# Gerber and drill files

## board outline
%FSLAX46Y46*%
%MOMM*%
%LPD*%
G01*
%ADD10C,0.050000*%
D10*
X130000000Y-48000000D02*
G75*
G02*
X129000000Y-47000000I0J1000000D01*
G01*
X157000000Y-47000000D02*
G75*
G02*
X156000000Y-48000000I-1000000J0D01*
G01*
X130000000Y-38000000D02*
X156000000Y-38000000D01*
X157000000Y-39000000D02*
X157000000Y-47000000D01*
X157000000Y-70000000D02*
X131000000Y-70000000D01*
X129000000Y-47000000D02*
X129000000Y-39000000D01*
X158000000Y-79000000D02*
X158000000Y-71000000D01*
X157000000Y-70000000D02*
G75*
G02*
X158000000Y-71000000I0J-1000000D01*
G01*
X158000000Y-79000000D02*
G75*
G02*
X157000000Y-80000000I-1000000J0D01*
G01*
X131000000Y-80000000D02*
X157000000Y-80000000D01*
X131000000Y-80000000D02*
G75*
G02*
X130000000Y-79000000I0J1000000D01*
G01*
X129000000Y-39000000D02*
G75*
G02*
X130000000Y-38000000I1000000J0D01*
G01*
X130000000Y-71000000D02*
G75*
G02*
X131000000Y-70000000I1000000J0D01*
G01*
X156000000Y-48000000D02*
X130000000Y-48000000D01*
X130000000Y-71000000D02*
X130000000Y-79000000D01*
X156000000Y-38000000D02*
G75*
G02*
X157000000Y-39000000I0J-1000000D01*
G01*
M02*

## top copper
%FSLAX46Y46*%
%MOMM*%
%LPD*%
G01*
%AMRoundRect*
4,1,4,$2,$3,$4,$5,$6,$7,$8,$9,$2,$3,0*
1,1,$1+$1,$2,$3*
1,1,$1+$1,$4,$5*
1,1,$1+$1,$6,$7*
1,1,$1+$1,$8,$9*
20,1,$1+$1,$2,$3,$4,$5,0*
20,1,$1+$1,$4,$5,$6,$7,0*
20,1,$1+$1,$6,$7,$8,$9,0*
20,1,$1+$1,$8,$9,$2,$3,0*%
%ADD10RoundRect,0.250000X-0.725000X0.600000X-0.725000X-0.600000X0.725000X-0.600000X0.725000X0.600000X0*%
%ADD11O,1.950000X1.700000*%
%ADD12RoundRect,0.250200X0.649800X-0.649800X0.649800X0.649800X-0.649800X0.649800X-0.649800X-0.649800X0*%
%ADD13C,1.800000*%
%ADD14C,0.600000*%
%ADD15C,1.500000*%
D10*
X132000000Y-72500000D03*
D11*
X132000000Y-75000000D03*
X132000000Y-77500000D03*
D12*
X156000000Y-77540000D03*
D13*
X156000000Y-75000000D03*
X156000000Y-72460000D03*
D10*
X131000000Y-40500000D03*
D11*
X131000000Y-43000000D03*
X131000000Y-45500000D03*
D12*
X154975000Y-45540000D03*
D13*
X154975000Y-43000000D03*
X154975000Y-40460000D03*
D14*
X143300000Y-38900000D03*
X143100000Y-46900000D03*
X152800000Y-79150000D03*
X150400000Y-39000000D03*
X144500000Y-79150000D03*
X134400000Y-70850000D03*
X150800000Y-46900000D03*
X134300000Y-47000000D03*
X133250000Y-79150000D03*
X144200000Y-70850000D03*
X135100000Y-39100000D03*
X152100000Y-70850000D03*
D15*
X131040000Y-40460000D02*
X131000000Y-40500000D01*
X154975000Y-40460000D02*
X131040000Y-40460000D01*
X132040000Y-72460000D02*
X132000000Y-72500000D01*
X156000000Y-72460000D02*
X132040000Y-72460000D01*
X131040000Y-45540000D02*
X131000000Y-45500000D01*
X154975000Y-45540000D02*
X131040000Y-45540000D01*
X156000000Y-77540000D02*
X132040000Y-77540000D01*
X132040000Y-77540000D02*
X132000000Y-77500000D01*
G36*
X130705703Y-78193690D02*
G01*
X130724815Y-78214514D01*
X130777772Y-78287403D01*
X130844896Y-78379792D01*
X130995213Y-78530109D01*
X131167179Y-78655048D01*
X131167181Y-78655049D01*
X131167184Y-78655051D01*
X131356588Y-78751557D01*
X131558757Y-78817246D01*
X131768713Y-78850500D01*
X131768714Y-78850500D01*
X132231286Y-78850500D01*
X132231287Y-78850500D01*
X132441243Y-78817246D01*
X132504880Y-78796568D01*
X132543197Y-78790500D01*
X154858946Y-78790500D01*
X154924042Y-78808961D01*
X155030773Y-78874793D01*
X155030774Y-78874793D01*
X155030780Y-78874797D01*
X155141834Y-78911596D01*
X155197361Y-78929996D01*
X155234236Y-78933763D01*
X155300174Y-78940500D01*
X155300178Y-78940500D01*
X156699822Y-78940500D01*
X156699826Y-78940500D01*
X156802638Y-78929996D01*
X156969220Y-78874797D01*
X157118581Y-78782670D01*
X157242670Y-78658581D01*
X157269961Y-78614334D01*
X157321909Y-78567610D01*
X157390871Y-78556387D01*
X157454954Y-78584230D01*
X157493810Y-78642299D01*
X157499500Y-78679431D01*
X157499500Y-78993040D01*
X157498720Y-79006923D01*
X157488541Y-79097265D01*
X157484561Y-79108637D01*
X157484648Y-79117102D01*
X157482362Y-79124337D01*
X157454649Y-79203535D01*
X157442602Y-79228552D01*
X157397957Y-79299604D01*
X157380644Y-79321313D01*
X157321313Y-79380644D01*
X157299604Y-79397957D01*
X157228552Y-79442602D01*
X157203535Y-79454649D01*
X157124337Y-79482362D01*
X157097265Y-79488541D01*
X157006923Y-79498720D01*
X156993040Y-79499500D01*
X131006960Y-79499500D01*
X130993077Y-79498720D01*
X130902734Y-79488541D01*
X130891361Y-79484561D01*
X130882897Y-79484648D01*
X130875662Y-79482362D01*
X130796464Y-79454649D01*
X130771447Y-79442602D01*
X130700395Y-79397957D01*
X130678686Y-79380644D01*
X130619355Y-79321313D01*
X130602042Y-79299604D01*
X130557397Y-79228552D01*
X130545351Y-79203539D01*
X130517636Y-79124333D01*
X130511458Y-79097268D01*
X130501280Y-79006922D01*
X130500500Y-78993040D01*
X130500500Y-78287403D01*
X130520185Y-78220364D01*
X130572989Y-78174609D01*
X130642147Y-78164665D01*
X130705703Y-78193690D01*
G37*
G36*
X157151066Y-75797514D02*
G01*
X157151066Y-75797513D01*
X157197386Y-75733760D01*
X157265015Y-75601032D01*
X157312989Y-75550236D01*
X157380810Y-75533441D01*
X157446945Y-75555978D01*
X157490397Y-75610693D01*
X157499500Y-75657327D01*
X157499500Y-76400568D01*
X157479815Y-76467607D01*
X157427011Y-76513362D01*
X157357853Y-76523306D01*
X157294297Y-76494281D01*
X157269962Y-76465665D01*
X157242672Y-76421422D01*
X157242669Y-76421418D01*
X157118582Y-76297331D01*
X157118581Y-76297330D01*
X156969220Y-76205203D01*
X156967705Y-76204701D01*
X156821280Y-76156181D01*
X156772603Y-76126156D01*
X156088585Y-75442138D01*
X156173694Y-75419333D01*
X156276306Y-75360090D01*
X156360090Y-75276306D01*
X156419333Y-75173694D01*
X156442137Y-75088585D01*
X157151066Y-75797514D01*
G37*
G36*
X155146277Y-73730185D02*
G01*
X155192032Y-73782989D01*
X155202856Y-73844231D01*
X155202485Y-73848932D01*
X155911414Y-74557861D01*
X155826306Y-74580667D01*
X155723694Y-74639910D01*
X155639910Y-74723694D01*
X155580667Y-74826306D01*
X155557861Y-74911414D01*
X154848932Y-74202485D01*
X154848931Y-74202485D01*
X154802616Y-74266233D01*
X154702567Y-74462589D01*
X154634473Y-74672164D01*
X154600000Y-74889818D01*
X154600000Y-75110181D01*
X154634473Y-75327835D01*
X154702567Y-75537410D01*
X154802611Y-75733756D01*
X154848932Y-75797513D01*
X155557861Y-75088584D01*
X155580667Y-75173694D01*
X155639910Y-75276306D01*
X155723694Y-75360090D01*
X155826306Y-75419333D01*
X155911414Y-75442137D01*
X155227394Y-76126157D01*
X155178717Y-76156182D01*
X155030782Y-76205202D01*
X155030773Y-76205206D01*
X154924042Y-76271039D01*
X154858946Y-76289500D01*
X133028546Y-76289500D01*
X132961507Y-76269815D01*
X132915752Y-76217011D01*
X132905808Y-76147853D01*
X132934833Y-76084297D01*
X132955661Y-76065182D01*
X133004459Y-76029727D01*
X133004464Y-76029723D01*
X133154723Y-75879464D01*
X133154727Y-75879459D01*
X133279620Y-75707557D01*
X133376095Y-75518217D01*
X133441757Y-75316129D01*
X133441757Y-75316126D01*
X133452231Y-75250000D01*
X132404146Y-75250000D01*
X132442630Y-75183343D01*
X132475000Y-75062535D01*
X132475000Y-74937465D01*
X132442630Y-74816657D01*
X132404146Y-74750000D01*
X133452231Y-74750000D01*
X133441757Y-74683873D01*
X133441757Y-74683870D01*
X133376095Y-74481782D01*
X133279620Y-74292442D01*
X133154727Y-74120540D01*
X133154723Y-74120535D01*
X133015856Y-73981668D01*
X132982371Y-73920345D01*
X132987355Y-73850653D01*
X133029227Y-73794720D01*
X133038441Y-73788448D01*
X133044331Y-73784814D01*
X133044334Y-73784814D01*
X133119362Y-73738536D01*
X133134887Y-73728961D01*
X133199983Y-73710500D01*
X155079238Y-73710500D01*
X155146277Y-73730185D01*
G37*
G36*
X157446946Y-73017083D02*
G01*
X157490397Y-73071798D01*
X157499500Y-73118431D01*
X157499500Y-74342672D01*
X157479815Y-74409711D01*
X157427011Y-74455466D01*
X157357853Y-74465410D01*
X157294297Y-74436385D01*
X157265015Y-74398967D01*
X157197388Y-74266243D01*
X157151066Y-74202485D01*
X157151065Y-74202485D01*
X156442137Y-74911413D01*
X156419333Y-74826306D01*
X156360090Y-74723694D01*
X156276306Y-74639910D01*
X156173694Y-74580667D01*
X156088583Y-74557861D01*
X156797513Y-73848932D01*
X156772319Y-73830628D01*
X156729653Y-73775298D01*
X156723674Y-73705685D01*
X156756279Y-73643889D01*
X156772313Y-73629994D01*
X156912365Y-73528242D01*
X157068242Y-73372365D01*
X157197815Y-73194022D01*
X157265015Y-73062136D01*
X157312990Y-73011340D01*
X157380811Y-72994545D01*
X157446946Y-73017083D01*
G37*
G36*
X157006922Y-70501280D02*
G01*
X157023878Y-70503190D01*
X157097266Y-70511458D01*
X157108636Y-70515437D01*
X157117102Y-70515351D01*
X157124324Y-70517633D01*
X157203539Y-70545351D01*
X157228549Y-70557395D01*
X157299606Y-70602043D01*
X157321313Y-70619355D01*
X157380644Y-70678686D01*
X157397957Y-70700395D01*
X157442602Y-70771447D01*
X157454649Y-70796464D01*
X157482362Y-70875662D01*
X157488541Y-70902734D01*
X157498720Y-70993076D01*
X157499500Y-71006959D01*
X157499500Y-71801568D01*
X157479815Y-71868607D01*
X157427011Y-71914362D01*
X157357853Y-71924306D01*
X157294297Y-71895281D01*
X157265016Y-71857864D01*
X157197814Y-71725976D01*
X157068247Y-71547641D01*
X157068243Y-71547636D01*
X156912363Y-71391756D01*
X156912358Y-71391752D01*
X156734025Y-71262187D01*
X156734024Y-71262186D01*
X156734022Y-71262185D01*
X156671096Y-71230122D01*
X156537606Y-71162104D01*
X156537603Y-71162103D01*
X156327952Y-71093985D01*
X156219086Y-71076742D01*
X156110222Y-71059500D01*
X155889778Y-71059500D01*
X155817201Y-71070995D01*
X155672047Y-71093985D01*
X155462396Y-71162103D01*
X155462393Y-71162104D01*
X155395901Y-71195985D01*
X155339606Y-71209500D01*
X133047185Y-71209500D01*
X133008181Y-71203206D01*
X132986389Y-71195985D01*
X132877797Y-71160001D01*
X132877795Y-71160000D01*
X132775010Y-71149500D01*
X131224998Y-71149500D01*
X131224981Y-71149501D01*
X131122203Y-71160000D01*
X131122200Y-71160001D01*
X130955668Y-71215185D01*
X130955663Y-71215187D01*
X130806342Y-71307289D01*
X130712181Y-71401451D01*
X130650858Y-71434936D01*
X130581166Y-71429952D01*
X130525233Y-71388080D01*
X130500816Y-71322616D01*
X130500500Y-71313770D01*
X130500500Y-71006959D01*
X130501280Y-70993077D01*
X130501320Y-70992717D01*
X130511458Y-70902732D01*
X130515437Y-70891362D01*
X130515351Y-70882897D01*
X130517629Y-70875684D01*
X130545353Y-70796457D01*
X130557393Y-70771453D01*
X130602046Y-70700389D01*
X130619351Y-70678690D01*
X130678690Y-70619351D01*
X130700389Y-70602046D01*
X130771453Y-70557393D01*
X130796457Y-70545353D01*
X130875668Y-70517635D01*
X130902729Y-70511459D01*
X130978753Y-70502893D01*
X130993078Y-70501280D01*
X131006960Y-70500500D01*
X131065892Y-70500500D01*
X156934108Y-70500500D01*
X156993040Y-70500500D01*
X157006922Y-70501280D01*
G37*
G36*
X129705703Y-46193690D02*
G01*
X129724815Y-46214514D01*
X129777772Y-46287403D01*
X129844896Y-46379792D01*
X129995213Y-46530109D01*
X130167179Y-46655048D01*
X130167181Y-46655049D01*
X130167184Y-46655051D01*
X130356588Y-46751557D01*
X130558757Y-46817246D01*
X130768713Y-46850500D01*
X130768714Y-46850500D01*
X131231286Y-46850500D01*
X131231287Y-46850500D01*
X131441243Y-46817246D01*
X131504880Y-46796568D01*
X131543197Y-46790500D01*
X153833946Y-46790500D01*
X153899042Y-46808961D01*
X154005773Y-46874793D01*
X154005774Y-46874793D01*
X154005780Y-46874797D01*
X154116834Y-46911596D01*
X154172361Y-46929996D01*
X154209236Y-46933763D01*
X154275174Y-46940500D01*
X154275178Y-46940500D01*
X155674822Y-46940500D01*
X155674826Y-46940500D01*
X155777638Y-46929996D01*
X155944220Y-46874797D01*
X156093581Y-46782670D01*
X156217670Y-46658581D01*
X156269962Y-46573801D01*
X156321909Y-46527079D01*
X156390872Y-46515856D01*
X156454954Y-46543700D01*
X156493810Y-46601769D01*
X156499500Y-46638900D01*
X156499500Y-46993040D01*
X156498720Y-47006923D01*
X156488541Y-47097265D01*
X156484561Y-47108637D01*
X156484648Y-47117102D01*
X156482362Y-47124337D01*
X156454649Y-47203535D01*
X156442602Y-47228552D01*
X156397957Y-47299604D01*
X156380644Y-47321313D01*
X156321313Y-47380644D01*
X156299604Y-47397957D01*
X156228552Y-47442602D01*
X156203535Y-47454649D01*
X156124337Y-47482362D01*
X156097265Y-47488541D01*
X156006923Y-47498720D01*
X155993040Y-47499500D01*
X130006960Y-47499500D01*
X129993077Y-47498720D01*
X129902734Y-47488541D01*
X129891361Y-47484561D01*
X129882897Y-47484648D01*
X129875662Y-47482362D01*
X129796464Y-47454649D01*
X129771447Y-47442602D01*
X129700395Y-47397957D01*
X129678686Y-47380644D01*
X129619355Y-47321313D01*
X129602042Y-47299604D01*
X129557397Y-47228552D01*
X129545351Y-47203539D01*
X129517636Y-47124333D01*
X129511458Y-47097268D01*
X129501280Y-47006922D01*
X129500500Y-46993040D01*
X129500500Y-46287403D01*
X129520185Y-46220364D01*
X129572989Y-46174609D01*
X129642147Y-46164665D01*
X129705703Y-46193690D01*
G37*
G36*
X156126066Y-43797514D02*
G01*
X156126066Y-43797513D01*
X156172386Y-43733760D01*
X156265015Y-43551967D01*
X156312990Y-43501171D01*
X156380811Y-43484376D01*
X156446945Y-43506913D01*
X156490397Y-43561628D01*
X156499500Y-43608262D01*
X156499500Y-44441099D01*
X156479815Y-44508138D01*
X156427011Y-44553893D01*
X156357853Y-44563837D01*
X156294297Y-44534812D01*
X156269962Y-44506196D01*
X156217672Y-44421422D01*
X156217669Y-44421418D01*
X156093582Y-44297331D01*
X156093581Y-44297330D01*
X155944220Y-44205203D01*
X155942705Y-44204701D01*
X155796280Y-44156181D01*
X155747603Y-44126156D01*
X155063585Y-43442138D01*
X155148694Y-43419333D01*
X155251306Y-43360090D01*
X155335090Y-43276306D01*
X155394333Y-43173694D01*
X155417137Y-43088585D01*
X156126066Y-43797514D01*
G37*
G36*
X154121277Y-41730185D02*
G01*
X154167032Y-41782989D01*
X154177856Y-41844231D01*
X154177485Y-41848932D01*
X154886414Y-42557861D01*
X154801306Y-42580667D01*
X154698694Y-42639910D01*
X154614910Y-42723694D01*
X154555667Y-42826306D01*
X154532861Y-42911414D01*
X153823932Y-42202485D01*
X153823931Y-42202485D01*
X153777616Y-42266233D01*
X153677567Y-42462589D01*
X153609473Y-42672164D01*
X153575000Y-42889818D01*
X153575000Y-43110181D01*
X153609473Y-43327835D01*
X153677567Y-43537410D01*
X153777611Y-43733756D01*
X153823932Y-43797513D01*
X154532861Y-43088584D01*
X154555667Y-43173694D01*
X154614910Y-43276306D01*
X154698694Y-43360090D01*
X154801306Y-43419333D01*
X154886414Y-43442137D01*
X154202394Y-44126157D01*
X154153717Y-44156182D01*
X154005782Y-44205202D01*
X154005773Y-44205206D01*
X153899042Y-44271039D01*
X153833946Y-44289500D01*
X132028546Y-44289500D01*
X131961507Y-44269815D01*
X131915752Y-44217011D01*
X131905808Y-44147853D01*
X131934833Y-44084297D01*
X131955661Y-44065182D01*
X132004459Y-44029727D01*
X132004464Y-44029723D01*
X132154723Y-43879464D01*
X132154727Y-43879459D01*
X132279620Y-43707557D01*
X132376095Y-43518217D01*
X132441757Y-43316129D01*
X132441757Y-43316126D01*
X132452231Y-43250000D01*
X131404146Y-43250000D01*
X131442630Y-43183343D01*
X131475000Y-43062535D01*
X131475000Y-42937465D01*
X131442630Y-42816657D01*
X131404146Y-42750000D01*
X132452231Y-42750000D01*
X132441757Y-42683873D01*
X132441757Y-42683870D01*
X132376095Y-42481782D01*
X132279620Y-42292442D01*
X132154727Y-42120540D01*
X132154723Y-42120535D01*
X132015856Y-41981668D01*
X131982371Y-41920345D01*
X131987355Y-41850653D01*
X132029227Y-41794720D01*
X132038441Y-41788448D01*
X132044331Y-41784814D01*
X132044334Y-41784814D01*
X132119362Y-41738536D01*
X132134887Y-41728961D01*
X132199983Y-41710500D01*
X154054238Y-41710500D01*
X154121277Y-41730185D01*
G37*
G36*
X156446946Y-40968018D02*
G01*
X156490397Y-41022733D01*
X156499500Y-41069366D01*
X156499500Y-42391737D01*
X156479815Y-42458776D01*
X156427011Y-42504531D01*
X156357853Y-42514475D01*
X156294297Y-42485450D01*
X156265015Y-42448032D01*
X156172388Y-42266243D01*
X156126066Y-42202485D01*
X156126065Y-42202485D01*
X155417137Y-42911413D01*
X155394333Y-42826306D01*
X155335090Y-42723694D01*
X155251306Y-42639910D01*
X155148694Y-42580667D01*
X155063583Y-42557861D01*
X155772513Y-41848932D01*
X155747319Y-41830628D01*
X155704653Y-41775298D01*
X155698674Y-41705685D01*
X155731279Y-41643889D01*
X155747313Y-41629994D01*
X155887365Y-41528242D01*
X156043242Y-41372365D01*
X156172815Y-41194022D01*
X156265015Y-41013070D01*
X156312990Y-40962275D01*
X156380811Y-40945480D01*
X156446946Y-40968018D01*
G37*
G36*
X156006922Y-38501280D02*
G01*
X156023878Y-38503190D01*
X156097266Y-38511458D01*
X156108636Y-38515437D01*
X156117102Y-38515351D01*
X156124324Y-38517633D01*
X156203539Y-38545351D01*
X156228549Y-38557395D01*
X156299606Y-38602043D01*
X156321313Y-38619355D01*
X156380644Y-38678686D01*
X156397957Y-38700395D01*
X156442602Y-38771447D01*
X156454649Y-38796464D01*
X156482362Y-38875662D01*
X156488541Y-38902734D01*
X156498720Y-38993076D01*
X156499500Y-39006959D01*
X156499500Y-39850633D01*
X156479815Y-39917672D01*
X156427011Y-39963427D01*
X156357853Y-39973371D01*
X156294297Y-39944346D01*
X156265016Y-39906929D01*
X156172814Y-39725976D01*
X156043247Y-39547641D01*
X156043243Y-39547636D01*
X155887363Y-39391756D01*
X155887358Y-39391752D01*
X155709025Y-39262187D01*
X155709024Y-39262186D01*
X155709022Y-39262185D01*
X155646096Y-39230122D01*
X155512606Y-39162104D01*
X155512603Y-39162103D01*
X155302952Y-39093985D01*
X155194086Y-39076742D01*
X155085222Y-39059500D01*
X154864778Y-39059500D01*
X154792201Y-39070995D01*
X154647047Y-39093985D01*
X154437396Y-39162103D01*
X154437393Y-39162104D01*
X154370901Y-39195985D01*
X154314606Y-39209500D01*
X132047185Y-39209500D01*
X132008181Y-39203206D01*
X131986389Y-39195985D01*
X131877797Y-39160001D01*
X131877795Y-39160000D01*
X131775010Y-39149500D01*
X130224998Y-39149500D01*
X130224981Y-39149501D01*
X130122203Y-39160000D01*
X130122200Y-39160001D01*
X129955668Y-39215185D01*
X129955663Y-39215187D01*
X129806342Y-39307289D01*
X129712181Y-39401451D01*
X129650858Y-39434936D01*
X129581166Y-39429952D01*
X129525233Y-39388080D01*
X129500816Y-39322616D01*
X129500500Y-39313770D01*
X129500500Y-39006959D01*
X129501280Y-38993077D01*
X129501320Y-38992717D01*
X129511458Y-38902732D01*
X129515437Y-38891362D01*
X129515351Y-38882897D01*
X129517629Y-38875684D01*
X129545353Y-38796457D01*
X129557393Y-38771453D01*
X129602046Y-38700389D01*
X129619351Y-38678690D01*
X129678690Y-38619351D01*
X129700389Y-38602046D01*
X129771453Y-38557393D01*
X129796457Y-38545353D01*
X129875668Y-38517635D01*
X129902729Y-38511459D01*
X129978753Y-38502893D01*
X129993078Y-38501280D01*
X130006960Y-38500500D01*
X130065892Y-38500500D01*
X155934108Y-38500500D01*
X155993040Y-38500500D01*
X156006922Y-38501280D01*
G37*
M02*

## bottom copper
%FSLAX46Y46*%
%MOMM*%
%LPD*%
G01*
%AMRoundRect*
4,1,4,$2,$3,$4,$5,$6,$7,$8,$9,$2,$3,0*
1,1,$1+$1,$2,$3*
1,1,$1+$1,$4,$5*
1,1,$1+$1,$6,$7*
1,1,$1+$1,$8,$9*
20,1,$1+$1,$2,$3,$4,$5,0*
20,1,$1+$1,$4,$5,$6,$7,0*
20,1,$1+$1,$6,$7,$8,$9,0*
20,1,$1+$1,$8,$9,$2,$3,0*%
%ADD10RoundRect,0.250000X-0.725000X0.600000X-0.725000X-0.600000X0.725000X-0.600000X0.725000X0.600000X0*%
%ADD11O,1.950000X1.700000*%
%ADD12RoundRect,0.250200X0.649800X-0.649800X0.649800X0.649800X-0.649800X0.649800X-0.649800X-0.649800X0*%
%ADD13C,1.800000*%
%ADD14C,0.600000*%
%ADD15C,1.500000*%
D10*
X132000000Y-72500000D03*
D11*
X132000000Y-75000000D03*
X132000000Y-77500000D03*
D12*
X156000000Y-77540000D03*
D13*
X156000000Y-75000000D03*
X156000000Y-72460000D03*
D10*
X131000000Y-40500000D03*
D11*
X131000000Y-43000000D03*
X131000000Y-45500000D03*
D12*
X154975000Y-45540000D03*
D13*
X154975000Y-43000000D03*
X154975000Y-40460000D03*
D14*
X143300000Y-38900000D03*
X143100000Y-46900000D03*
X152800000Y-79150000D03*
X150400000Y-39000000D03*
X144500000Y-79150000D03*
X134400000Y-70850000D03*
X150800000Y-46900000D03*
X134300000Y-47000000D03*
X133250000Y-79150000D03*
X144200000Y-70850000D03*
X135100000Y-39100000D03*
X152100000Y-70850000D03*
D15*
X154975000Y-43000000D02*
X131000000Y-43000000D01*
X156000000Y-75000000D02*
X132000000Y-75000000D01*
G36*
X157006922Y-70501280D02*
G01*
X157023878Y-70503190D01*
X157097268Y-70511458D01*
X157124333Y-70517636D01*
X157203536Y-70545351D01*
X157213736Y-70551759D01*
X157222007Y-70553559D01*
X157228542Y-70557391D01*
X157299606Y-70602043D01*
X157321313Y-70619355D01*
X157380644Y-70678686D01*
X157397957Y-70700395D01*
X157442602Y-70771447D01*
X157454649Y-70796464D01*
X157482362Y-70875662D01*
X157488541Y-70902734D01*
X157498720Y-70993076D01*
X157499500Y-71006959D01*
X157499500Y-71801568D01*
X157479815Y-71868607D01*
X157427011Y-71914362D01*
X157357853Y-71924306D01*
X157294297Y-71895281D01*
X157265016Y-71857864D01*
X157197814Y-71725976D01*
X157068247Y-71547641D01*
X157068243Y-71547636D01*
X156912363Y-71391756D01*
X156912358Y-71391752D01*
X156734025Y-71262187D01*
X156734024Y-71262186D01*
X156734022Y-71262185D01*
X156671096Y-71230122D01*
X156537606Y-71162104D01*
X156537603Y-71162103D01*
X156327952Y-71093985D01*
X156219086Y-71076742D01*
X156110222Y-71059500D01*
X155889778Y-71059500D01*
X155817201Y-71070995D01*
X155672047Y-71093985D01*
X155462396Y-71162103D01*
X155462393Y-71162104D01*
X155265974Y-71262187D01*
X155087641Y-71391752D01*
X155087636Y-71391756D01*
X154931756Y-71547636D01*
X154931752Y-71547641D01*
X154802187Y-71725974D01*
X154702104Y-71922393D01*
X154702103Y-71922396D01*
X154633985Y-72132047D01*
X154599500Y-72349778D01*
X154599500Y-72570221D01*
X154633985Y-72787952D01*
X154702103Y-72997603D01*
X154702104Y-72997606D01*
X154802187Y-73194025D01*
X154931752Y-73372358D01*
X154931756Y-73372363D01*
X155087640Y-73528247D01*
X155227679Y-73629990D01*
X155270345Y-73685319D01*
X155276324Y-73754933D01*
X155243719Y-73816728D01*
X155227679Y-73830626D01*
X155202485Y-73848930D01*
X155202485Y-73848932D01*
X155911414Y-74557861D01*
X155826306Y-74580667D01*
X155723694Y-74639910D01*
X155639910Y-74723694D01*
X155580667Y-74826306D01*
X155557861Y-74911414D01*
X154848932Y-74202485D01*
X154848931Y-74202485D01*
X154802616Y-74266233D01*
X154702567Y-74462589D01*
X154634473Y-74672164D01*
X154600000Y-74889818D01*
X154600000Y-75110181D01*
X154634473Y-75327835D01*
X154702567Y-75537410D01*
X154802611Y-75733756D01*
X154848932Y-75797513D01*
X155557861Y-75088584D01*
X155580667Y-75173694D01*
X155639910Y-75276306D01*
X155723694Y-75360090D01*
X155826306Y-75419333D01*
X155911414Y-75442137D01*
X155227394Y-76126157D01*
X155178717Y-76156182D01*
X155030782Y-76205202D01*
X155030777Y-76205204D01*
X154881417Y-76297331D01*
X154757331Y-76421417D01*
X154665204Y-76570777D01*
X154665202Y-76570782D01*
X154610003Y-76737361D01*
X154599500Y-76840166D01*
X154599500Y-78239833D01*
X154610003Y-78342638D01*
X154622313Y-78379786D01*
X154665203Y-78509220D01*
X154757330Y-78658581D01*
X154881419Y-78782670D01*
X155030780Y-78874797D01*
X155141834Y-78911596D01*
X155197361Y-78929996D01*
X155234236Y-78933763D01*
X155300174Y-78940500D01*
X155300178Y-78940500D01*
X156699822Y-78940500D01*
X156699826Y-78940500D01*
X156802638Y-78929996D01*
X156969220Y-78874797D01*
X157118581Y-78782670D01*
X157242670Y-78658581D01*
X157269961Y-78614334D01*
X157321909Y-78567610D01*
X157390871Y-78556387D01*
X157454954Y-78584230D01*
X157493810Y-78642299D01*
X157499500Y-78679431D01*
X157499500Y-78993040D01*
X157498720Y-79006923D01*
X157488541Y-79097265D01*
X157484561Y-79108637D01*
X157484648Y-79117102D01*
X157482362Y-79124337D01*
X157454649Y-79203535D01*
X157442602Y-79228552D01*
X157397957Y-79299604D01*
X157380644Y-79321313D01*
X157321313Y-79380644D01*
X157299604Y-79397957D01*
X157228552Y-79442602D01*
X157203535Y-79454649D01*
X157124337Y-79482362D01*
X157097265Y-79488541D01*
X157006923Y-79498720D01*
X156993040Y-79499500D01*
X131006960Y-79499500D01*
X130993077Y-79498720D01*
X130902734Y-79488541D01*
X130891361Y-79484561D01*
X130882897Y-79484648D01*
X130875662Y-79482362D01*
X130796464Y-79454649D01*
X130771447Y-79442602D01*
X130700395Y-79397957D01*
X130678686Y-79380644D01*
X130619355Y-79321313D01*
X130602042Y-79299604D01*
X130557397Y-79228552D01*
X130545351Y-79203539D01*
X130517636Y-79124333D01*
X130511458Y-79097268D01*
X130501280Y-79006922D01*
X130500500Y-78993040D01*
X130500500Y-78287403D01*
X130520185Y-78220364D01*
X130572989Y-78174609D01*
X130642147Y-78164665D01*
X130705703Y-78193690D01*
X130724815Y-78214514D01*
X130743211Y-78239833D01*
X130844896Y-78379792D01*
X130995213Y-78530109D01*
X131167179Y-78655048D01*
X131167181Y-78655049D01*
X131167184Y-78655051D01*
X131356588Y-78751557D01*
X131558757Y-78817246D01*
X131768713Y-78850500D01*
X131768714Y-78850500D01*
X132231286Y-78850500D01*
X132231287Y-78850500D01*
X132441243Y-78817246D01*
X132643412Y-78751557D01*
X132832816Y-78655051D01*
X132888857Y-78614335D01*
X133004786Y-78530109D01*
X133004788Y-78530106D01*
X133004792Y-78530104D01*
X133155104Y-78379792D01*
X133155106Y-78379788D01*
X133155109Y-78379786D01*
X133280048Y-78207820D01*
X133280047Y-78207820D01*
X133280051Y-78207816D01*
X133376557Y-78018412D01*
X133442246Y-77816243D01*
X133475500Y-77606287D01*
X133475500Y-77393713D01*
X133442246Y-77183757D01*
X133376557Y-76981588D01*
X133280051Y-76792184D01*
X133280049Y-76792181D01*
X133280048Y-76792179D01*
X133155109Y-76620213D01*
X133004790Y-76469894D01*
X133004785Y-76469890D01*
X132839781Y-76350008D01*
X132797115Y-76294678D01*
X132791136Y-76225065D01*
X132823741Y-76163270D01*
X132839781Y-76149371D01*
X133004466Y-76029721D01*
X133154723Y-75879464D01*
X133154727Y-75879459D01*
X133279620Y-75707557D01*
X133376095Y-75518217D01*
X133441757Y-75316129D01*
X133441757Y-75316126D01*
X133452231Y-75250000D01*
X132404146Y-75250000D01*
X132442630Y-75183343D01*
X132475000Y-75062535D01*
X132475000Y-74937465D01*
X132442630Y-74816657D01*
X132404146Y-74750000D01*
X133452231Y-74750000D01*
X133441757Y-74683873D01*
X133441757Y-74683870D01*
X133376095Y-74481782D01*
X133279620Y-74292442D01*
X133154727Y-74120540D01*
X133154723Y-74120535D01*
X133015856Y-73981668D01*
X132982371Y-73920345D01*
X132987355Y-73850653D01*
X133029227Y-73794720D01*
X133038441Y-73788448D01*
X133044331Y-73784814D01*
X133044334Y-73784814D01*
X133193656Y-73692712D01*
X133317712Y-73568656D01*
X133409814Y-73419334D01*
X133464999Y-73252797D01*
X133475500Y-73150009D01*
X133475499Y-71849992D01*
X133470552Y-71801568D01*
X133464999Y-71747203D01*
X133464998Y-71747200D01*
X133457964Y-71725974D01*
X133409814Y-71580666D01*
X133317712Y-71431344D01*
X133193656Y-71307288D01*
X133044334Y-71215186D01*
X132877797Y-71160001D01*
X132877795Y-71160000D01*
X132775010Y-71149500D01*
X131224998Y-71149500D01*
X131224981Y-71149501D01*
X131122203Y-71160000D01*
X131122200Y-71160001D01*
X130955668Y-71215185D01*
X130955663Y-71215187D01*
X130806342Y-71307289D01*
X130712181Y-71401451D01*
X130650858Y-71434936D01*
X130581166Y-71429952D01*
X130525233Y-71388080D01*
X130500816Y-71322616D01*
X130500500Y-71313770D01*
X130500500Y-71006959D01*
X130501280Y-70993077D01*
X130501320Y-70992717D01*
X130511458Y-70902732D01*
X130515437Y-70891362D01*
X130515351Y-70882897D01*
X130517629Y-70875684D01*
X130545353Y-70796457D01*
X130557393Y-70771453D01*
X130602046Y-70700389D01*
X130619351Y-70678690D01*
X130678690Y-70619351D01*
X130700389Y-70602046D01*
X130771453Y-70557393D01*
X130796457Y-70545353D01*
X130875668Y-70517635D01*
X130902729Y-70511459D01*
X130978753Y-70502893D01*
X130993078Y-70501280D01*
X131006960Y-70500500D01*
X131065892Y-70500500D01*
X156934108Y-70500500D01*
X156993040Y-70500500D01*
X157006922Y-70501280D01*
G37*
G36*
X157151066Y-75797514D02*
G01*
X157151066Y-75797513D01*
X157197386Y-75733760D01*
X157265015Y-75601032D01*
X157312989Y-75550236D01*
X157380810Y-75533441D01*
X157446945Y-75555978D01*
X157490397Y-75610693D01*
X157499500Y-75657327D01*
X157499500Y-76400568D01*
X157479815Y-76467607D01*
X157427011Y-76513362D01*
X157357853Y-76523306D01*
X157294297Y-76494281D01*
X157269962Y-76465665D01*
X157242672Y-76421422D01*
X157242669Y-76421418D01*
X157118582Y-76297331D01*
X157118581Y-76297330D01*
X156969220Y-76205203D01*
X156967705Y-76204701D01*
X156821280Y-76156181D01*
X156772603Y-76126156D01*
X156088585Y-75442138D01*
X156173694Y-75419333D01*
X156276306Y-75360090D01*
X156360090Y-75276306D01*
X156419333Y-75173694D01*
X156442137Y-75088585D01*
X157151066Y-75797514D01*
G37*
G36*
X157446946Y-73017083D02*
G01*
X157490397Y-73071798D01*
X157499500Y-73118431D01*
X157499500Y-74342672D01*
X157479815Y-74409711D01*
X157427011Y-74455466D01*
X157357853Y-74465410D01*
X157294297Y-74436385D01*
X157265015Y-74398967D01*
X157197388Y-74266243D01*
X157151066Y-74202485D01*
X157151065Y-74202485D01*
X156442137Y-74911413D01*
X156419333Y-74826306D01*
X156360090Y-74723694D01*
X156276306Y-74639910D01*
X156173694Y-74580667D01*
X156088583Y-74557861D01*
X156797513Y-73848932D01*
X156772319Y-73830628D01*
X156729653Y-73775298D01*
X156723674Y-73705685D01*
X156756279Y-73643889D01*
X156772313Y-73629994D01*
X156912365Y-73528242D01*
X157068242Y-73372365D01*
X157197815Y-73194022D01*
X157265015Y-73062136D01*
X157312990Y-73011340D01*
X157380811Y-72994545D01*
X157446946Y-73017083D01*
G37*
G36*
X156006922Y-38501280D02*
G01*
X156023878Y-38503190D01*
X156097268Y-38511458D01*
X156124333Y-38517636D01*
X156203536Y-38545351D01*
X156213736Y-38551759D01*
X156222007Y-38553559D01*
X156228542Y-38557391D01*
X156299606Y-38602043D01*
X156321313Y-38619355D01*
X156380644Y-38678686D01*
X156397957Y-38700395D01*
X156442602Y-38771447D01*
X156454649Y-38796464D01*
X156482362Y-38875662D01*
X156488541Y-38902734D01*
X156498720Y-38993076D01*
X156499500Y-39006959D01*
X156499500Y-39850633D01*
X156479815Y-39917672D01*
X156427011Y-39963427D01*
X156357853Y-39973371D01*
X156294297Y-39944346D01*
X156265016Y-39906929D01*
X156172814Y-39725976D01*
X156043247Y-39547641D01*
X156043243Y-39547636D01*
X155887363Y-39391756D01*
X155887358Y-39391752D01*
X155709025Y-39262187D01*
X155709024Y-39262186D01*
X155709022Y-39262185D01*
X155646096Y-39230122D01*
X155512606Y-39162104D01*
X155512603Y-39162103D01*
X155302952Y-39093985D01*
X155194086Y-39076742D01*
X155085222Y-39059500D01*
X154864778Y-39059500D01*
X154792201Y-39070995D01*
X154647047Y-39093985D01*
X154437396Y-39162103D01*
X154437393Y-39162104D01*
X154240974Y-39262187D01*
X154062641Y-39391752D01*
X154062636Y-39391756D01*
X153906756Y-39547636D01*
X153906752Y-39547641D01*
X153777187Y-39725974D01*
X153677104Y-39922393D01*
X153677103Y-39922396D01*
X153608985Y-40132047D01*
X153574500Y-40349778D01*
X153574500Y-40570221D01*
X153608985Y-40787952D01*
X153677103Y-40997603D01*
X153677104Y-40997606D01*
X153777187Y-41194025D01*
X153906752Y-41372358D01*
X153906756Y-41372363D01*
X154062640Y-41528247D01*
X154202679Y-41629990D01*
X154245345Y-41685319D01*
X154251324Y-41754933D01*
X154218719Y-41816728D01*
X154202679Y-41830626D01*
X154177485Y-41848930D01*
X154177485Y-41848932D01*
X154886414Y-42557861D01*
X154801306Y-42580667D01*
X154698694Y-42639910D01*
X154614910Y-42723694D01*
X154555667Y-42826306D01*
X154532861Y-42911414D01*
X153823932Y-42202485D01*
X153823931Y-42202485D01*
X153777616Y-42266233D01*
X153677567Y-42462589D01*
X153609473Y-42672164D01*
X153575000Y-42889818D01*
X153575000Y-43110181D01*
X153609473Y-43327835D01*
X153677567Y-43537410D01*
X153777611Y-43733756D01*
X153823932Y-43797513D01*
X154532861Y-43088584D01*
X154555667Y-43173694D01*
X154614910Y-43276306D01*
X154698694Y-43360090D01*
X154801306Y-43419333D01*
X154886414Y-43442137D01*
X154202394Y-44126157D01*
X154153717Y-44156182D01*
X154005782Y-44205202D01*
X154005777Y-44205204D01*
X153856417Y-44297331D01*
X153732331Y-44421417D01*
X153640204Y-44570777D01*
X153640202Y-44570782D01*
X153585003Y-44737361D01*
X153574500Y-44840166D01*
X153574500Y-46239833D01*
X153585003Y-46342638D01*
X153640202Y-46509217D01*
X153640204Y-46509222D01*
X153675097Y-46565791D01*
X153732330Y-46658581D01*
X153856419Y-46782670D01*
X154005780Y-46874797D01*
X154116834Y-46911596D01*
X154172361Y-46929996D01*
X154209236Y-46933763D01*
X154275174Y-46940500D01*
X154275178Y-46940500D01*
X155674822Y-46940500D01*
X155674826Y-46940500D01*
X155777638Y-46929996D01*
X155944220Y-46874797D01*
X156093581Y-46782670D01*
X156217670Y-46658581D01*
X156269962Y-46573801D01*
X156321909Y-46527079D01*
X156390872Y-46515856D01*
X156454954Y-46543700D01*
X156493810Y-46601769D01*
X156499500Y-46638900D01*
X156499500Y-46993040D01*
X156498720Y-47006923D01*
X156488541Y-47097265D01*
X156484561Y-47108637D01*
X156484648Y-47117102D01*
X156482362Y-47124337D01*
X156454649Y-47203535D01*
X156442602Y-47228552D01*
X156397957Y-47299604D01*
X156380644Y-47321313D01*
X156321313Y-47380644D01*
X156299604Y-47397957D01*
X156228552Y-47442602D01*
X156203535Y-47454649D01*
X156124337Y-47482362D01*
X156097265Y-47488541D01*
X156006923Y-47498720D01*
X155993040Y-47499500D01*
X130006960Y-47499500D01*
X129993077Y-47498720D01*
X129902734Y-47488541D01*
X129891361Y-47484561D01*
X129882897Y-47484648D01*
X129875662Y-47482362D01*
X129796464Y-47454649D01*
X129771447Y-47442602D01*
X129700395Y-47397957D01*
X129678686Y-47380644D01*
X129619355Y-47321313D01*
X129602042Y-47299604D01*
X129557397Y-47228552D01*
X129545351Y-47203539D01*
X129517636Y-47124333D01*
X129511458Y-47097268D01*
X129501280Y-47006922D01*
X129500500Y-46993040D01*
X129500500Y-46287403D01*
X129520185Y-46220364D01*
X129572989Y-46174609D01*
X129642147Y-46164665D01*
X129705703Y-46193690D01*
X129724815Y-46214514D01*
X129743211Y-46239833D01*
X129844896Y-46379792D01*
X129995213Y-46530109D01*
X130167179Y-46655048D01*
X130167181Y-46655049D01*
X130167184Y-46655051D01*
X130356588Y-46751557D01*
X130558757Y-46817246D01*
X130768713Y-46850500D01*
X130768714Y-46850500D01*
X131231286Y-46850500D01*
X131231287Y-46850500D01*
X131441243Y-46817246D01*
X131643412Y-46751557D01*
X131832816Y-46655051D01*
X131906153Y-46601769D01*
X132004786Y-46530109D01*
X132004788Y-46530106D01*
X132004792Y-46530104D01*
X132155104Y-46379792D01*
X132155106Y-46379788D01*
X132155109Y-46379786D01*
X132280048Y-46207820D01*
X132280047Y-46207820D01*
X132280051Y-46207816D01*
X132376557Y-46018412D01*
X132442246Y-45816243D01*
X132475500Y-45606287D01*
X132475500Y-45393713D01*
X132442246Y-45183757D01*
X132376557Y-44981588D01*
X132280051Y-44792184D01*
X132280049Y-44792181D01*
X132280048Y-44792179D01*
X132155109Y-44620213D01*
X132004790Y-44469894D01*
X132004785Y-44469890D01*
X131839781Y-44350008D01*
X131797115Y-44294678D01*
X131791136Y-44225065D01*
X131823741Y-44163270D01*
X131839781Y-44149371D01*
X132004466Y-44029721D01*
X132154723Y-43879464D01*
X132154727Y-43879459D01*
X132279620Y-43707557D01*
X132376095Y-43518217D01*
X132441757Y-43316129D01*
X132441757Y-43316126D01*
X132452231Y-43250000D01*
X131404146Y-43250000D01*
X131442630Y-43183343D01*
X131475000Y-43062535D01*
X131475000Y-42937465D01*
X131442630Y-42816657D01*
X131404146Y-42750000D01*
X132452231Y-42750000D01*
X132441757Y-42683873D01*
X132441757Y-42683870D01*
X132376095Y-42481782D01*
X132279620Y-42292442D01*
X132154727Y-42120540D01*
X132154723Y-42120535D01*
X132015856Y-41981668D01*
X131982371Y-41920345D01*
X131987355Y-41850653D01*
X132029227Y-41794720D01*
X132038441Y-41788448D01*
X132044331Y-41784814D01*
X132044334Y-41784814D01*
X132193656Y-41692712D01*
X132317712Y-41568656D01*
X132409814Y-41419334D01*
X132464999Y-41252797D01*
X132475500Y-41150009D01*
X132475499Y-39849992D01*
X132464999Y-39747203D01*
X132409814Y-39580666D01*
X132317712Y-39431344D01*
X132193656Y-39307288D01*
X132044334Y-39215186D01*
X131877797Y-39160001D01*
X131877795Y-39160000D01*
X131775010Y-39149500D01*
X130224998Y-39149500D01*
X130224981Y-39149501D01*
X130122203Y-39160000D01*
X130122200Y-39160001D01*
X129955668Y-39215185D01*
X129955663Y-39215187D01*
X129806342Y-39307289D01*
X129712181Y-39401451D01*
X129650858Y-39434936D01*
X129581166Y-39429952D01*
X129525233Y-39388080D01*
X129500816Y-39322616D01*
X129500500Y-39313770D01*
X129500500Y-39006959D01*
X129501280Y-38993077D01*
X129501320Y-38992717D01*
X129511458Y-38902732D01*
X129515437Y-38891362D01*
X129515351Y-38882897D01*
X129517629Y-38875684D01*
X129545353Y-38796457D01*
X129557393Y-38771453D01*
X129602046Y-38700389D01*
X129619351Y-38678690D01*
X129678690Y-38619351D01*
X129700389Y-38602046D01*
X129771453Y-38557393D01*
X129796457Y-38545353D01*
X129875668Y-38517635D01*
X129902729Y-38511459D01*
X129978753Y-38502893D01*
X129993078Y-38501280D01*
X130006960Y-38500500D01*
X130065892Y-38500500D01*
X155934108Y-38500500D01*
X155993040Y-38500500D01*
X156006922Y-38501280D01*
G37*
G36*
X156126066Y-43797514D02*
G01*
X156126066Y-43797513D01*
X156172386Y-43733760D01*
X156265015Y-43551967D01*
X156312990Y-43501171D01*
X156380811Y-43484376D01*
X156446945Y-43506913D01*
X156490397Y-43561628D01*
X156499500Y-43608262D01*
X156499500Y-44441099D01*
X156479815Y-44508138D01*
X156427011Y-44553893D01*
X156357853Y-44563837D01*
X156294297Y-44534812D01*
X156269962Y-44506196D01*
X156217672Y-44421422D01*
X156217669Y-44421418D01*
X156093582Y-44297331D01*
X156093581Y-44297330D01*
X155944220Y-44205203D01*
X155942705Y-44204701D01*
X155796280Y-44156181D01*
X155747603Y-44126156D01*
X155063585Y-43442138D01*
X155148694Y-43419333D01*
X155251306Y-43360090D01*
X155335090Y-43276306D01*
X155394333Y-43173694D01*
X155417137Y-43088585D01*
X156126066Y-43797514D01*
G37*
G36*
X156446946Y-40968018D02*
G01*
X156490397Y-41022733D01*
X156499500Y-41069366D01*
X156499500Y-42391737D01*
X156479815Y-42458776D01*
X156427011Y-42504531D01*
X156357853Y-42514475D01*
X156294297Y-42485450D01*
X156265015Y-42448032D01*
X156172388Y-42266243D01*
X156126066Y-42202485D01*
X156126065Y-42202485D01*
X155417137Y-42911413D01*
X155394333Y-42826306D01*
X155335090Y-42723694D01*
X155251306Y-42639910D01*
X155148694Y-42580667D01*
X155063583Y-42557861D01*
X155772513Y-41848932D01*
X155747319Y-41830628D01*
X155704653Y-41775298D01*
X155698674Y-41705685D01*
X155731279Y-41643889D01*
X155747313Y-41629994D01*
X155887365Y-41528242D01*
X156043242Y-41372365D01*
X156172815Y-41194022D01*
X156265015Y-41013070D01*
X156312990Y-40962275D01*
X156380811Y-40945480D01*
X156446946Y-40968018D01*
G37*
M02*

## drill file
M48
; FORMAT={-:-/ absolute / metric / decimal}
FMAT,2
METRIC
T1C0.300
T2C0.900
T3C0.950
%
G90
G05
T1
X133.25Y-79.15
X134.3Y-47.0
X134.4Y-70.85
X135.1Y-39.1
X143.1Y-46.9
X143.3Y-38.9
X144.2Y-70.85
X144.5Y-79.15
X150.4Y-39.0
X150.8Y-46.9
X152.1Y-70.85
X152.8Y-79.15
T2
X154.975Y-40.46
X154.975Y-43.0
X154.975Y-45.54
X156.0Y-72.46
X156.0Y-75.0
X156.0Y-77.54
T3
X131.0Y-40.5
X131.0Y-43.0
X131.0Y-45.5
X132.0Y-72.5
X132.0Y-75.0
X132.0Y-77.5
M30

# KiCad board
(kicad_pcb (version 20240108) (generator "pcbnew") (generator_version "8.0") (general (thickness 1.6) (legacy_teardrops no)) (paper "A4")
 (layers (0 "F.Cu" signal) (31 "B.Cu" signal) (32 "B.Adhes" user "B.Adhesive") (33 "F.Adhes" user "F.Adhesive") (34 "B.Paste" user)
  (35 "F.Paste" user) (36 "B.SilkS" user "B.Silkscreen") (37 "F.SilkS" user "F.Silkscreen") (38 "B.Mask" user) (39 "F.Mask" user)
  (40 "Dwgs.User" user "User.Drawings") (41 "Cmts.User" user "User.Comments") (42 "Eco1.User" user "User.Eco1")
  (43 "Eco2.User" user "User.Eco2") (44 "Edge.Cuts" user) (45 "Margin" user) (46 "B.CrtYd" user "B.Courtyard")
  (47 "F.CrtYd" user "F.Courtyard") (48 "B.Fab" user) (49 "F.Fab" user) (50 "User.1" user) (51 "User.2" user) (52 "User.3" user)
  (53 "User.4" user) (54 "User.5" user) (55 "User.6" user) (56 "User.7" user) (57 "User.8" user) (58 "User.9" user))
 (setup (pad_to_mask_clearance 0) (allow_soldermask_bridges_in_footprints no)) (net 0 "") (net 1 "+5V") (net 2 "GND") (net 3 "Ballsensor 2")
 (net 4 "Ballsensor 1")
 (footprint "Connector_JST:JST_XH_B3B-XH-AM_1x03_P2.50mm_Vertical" (layer "F.Cu") (at 132 72.5 -90)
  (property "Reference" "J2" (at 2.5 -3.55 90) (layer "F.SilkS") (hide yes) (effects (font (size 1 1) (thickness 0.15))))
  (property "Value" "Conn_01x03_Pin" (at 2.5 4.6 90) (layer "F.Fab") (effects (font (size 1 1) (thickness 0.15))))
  (pad "1" thru_hole roundrect (at 0 0 270) (size 1.7 1.95) (drill 0.95) (layers "*.Cu" "*.Mask") (remove_unused_layers no)
   (roundrect_rratio 0.147059) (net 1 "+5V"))
  (pad "2" thru_hole oval (at 2.5 0 270) (size 1.7 1.95) (drill 0.95) (layers "*.Cu" "*.Mask") (remove_unused_layers no) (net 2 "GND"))
  (pad "3" thru_hole oval (at 5 0 270) (size 1.7 1.95) (drill 0.95) (layers "*.Cu" "*.Mask") (remove_unused_layers no)
   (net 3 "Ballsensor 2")))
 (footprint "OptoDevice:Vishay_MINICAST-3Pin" (layer "F.Cu") (at 156 77.54 90)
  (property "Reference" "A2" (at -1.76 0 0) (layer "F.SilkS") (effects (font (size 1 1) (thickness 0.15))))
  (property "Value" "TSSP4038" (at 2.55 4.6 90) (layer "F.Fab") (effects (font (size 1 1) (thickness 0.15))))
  (pad "1" thru_hole roundrect (at 0 0 90) (size 1.8 1.8) (drill 0.9) (layers "*.Cu" "*.Mask") (remove_unused_layers no)
   (roundrect_rratio 0.139) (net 3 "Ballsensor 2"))
  (pad "2" thru_hole circle (at 2.54 0 90) (size 1.8 1.8) (drill 0.9) (layers "*.Cu" "*.Mask") (remove_unused_layers no) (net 2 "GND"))
  (pad "3" thru_hole circle (at 5.08 0 90) (size 1.8 1.8) (drill 0.9) (layers "*.Cu" "*.Mask") (remove_unused_layers no) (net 1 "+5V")))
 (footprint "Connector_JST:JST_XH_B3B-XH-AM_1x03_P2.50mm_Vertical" (layer "F.Cu") (at 131 40.5 -90)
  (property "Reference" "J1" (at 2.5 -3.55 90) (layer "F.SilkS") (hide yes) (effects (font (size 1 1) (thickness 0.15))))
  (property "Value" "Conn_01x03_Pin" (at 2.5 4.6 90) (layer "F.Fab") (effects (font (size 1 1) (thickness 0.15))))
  (pad "1" thru_hole roundrect (at 0 0 270) (size 1.7 1.95) (drill 0.95) (layers "*.Cu" "*.Mask") (remove_unused_layers no)
   (roundrect_rratio 0.147059) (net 1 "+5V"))
  (pad "2" thru_hole oval (at 2.5 0 270) (size 1.7 1.95) (drill 0.95) (layers "*.Cu" "*.Mask") (remove_unused_layers no) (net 2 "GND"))
  (pad "3" thru_hole oval (at 5 0 270) (size 1.7 1.95) (drill 0.95) (layers "*.Cu" "*.Mask") (remove_unused_layers no)
   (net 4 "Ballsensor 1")))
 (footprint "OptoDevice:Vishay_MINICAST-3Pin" (layer "F.Cu") (at 154.975 45.54 90)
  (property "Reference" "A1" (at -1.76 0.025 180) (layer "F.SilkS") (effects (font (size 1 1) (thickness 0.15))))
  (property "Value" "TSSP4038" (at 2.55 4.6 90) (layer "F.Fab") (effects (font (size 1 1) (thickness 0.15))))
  (pad "1" thru_hole roundrect (at 0 0 90) (size 1.8 1.8) (drill 0.9) (layers "*.Cu" "*.Mask") (remove_unused_layers no)
   (roundrect_rratio 0.139) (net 4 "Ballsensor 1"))
  (pad "2" thru_hole circle (at 2.54 0 90) (size 1.8 1.8) (drill 0.9) (layers "*.Cu" "*.Mask") (remove_unused_layers no) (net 2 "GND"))
  (pad "3" thru_hole circle (at 5.08 0 90) (size 1.8 1.8) (drill 0.9) (layers "*.Cu" "*.Mask") (remove_unused_layers no) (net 1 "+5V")))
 (gr_arc (start 130 48) (mid 129.292893 47.707107) (end 129 47) (stroke (width 0.05) (type default)) (layer "Edge.Cuts"))
 (gr_arc (start 157 47) (mid 156.707107 47.707107) (end 156 48) (stroke (width 0.05) (type default)) (layer "Edge.Cuts"))
 (gr_line (start 130 38) (end 156 38) (stroke (width 0.05) (type default)) (layer "Edge.Cuts"))
 (gr_line (start 157 39) (end 157 47) (stroke (width 0.05) (type default)) (layer "Edge.Cuts"))
 (gr_line (start 157 70) (end 131 70) (stroke (width 0.05) (type default)) (layer "Edge.Cuts"))
 (gr_line (start 129 47) (end 129 39) (stroke (width 0.05) (type default)) (layer "Edge.Cuts"))
 (gr_line (start 158 79) (end 158 71) (stroke (width 0.05) (type default)) (layer "Edge.Cuts"))
 (gr_arc (start 157 70) (mid 157.707107 70.292893) (end 158 71) (stroke (width 0.05) (type default)) (layer "Edge.Cuts"))
 (gr_arc (start 158 79) (mid 157.707107 79.707107) (end 157 80) (stroke (width 0.05) (type default)) (layer "Edge.Cuts"))
 (gr_line (start 131 80) (end 157 80) (stroke (width 0.05) (type default)) (layer "Edge.Cuts"))
 (gr_arc (start 131 80) (mid 130.292893 79.707107) (end 130 79) (stroke (width 0.05) (type default)) (layer "Edge.Cuts"))
 (gr_arc (start 129 39) (mid 129.292893 38.292893) (end 130 38) (stroke (width 0.05) (type default)) (layer "Edge.Cuts"))
 (gr_arc (start 130 71) (mid 130.292893 70.292893) (end 131 70) (stroke (width 0.05) (type default)) (layer "Edge.Cuts"))
 (gr_line (start 156 48) (end 130 48) (stroke (width 0.05) (type default)) (layer "Edge.Cuts"))
 (gr_line (start 130 71) (end 130 79) (stroke (width 0.05) (type default)) (layer "Edge.Cuts"))
 (gr_arc (start 156 38) (mid 156.707107 38.292893) (end 157 39) (stroke (width 0.05) (type default)) (layer "Edge.Cuts"))
 (segment (start 131.04 40.46) (end 131 40.5) (width 1.5) (layer "F.Cu") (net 1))
 (segment (start 154.975 40.46) (end 131.04 40.46) (width 1.5) (layer "F.Cu") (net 1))
 (segment (start 132.04 72.46) (end 132 72.5) (width 1.5) (layer "F.Cu") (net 1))
 (segment (start 156 72.46) (end 132.04 72.46) (width 1.5) (layer "F.Cu") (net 1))
 (via (at 143.3 38.9) (size 0.6) (drill 0.3) (layers "F.Cu" "B.Cu") (free yes) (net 2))
 (via (at 143.1 46.9) (size 0.6) (drill 0.3) (layers "F.Cu" "B.Cu") (free yes) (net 2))
 (via (at 152.8 79.15) (size 0.6) (drill 0.3) (layers "F.Cu" "B.Cu") (free yes) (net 2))
 (via (at 150.4 39) (size 0.6) (drill 0.3) (layers "F.Cu" "B.Cu") (free yes) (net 2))
 (via (at 144.5 79.15) (size 0.6) (drill 0.3) (layers "F.Cu" "B.Cu") (free yes) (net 2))
 (via (at 134.4 70.85) (size 0.6) (drill 0.3) (layers "F.Cu" "B.Cu") (free yes) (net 2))
 (via (at 150.8 46.9) (size 0.6) (drill 0.3) (layers "F.Cu" "B.Cu") (free yes) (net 2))
 (via (at 134.3 47) (size 0.6) (drill 0.3) (layers "F.Cu" "B.Cu") (free yes) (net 2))
 (via (at 133.25 79.15) (size 0.6) (drill 0.3) (layers "F.Cu" "B.Cu") (free yes) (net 2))
 (via (at 144.2 70.85) (size 0.6) (drill 0.3) (layers "F.Cu" "B.Cu") (free yes) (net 2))
 (via (at 135.1 39.1) (size 0.6) (drill 0.3) (layers "F.Cu" "B.Cu") (free yes) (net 2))
 (via (at 152.1 70.85) (size 0.6) (drill 0.3) (layers "F.Cu" "B.Cu") (free yes) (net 2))
 (segment (start 154.975 43) (end 131 43) (width 1.5) (layer "B.Cu") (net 2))
 (segment (start 156 75) (end 132 75) (width 1.5) (layer "B.Cu") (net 2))
 (segment (start 131.04 45.54) (end 131 45.5) (width 1.5) (layer "F.Cu") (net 4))
 (segment (start 154.975 45.54) (end 131.04 45.54) (width 1.5) (layer "F.Cu") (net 4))
 (segment (start 156 77.54) (end 132.04 77.54) (width 1.5) (layer "F.Cu") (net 3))
 (segment (start 132.04 77.54) (end 132 77.5) (width 1.5) (layer "F.Cu") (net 3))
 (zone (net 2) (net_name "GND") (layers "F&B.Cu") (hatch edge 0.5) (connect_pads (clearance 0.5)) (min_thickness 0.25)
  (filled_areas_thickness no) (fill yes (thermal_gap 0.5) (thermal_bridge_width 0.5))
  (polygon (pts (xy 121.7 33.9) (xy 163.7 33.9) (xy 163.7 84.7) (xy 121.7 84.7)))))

